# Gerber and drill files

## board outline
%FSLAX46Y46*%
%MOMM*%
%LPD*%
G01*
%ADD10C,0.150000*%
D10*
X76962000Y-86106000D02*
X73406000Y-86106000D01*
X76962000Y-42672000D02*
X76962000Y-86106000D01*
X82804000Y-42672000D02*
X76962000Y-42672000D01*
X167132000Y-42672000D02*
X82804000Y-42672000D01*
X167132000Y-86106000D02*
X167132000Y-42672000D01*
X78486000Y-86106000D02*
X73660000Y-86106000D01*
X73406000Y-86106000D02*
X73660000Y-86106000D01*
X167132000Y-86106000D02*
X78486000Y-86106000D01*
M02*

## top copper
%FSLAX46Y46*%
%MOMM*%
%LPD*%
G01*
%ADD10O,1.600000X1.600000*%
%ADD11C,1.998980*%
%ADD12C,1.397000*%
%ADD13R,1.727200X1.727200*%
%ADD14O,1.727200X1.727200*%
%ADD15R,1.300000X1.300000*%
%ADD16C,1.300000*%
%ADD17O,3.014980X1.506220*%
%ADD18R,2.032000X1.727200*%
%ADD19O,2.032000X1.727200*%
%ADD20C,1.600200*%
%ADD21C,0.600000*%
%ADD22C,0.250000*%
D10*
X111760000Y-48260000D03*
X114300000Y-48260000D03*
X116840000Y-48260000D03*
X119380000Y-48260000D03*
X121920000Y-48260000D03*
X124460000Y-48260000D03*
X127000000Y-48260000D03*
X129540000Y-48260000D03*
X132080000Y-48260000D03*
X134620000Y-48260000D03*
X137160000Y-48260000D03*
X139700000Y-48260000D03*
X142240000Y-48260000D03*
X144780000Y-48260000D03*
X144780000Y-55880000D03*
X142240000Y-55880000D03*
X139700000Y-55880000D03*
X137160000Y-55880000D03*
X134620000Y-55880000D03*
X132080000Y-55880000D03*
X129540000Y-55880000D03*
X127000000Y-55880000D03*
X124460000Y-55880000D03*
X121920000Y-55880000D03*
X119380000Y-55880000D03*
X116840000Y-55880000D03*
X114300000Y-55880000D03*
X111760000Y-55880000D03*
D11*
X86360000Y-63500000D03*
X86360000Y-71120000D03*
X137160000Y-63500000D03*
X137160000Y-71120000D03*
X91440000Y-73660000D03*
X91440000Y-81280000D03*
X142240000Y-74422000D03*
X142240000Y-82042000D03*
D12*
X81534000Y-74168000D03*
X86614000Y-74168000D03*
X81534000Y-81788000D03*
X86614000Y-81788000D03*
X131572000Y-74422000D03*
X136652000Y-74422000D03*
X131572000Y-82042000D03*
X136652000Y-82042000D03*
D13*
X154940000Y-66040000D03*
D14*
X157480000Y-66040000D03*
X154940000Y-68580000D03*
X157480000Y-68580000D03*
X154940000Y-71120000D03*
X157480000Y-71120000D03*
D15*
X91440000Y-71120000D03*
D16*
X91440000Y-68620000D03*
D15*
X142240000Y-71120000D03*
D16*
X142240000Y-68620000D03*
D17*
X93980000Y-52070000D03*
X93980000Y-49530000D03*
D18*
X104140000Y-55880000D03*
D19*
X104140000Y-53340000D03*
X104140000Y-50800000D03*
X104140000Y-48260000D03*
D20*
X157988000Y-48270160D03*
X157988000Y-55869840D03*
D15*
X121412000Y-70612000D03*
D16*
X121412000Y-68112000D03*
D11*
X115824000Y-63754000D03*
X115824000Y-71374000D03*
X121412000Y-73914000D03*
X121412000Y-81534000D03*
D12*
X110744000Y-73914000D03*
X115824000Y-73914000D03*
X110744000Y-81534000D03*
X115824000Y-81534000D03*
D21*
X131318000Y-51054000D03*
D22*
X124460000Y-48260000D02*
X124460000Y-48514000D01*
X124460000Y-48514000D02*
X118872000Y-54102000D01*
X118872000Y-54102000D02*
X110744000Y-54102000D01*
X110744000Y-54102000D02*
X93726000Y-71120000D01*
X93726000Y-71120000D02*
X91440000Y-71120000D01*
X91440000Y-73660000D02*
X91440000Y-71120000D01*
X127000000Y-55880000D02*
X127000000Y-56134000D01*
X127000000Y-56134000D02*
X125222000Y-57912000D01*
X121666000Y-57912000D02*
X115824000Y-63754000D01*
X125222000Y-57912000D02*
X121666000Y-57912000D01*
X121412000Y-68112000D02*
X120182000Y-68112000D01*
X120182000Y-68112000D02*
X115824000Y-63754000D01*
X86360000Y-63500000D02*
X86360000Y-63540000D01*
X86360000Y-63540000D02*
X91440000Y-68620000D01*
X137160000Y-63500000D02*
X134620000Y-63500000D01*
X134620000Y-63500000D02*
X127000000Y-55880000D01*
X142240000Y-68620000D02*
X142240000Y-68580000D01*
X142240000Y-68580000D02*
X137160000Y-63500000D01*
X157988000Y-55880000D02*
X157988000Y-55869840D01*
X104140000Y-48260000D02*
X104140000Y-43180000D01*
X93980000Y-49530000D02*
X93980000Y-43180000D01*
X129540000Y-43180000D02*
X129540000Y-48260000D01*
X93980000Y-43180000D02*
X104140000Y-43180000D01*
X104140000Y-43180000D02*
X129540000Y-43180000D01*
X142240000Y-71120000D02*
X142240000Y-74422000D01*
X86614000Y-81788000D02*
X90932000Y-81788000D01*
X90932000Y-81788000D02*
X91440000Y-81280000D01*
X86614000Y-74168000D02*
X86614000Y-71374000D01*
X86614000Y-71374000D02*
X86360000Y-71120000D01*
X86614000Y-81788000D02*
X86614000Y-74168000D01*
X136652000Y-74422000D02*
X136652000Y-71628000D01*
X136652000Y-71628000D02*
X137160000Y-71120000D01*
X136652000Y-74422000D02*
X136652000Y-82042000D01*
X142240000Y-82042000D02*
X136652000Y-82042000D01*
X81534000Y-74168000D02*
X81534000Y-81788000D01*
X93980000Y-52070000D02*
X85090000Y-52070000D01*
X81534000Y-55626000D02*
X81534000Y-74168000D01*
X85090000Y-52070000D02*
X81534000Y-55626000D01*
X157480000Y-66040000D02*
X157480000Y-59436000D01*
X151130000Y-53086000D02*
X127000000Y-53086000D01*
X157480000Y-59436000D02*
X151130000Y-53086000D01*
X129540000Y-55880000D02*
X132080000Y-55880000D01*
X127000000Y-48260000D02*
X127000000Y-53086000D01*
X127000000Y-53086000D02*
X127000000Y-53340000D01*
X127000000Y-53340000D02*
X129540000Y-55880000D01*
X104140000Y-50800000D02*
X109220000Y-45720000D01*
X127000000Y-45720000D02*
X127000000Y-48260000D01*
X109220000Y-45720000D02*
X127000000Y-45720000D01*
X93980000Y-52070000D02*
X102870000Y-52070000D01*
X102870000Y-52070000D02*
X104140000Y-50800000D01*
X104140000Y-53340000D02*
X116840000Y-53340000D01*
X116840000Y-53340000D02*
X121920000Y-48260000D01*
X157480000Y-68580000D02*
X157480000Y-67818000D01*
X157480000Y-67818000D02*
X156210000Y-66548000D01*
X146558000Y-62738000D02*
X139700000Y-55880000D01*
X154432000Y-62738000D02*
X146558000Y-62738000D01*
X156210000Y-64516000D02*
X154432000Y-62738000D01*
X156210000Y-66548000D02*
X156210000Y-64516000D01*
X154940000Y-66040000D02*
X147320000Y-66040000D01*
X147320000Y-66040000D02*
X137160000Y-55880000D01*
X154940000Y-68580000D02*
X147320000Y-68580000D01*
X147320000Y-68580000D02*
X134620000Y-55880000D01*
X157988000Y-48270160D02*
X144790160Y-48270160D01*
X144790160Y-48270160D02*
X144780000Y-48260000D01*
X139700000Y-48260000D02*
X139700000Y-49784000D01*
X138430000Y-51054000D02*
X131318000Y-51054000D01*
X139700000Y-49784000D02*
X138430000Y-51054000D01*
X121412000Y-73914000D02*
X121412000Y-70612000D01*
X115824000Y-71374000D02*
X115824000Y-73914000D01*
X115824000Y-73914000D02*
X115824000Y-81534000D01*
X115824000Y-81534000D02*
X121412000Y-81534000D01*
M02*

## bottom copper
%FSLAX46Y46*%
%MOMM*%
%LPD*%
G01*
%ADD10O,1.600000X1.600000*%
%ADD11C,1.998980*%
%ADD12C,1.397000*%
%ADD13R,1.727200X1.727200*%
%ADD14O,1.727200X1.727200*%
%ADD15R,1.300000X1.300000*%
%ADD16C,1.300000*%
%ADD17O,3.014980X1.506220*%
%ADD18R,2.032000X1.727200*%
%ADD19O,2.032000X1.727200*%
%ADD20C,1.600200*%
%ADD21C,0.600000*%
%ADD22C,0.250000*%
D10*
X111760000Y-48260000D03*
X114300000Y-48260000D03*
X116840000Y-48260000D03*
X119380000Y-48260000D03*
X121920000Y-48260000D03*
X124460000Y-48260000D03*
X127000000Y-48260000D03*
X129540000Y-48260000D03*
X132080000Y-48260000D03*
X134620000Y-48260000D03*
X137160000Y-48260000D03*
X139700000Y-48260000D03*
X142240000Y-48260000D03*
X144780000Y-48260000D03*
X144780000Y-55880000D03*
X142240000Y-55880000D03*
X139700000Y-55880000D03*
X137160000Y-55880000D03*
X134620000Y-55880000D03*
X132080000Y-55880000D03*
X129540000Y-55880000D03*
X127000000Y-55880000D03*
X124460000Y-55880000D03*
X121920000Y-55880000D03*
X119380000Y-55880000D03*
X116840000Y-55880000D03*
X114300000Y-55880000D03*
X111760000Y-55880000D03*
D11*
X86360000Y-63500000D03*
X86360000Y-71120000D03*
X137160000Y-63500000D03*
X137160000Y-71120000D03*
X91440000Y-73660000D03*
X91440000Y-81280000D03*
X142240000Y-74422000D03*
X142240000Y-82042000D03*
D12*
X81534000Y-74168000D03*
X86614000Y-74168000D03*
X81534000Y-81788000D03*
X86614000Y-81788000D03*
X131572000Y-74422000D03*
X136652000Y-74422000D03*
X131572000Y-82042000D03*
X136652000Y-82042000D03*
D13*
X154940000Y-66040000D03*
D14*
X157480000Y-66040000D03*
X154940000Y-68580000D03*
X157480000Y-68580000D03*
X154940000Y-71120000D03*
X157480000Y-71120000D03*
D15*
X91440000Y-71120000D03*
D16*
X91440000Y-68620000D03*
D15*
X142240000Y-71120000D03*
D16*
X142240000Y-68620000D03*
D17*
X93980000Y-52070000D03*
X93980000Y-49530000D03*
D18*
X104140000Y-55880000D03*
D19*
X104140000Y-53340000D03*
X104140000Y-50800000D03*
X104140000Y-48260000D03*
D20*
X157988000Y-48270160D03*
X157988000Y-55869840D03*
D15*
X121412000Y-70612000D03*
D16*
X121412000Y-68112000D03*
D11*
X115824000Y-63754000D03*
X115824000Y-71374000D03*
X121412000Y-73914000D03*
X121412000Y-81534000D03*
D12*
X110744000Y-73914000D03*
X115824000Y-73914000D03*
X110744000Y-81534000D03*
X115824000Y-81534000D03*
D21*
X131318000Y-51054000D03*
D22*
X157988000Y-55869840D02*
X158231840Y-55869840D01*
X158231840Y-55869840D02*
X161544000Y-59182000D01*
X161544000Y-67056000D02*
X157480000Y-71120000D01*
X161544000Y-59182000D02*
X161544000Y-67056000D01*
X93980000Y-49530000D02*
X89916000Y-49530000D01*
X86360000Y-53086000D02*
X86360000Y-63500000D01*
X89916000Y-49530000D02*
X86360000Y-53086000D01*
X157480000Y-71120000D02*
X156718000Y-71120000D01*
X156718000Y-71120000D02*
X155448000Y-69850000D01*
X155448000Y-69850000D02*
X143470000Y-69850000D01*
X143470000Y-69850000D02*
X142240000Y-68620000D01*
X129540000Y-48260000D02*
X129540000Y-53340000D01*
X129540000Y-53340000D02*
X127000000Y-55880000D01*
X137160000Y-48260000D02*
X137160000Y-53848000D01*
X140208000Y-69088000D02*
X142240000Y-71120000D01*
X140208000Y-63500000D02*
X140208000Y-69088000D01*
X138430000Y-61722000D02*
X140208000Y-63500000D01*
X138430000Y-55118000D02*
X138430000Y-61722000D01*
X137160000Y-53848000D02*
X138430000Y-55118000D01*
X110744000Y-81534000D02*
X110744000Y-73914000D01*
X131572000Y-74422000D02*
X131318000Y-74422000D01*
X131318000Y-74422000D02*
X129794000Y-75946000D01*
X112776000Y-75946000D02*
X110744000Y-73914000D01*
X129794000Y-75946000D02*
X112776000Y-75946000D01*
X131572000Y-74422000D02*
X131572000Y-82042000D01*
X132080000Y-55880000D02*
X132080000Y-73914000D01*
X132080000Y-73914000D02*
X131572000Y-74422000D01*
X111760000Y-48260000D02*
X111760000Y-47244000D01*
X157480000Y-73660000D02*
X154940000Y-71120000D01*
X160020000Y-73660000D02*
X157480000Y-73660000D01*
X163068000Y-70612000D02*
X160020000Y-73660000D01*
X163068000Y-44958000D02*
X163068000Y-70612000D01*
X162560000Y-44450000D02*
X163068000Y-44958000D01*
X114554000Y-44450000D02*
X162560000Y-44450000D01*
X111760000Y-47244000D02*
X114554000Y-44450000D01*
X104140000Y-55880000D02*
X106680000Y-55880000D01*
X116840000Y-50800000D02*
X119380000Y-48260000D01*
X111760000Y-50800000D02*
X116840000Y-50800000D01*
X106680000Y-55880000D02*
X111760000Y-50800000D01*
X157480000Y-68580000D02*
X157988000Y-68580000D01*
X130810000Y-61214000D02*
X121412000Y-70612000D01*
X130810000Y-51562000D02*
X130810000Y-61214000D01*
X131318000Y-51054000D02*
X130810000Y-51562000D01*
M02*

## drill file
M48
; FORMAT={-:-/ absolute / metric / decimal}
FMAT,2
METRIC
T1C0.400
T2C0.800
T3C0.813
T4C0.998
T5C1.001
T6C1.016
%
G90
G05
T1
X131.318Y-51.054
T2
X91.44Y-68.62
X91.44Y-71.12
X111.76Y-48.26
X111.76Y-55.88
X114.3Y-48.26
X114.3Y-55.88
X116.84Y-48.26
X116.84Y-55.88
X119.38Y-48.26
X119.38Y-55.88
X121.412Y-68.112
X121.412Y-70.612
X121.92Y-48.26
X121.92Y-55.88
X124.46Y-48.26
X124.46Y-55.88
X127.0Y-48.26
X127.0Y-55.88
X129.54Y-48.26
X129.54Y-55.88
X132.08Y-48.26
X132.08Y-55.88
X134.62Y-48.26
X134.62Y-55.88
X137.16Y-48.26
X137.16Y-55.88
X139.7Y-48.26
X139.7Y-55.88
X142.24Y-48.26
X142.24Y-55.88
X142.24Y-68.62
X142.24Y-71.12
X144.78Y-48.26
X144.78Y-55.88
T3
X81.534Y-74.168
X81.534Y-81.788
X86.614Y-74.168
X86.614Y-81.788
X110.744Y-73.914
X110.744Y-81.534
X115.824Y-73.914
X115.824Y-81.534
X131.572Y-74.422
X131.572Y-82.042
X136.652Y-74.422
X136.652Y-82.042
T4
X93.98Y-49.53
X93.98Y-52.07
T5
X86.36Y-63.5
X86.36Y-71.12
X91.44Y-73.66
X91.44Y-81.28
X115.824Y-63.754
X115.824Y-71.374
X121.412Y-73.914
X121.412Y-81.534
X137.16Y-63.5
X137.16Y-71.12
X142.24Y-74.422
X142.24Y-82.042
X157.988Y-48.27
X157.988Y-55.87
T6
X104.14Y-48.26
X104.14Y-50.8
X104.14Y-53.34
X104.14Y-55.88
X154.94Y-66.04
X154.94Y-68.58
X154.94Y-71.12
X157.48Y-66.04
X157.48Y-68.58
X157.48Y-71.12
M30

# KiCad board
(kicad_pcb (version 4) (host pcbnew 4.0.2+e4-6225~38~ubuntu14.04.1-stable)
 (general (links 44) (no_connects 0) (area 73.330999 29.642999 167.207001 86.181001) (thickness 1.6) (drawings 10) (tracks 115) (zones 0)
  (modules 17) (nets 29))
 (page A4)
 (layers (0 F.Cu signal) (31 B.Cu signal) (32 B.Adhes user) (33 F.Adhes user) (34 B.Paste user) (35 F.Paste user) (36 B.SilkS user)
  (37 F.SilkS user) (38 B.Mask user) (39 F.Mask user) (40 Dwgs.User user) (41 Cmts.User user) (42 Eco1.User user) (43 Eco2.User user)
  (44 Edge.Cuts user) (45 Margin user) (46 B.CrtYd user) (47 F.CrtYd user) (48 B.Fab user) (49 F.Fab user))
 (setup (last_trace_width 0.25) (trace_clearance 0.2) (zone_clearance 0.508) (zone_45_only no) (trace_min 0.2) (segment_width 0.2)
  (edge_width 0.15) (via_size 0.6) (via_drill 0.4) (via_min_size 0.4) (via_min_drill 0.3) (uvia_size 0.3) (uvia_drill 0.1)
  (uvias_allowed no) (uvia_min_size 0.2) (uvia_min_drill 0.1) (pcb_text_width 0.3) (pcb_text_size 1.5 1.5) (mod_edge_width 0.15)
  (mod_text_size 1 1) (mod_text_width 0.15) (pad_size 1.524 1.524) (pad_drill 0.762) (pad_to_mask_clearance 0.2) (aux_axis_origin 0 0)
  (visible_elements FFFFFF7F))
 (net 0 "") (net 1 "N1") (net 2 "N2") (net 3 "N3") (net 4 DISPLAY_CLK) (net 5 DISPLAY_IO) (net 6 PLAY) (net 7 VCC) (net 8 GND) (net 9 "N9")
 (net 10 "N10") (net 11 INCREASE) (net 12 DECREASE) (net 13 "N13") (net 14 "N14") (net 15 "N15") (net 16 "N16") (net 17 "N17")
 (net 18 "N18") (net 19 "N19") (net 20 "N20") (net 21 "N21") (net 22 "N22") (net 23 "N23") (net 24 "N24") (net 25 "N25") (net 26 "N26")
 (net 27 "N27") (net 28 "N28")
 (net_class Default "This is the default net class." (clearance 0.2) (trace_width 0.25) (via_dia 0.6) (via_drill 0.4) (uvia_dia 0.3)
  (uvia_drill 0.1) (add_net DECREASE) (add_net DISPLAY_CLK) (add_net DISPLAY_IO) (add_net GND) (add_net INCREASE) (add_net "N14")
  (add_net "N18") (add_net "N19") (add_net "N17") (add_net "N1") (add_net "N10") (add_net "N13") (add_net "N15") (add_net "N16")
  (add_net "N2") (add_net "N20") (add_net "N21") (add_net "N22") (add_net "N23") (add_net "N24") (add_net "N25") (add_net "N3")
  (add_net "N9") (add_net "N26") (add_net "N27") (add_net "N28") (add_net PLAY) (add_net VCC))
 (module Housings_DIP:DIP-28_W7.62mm (layer B.Cu) (at 111.76 48.26 270)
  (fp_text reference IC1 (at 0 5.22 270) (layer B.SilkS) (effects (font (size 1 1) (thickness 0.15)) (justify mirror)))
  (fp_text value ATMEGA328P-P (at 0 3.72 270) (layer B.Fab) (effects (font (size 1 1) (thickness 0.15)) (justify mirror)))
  (pad 1 thru_hole oval (at 0 0 270) (size 1.6 1.6) (drill 0.8) (layers *.Cu *.Mask B.SilkS) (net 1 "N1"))
  (pad 2 thru_hole oval (at 0 -2.54 270) (size 1.6 1.6) (drill 0.8) (layers *.Cu *.Mask B.SilkS) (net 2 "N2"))
  (pad 3 thru_hole oval (at 0 -5.08 270) (size 1.6 1.6) (drill 0.8) (layers *.Cu *.Mask B.SilkS) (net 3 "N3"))
  (pad 4 thru_hole oval (at 0 -7.62 270) (size 1.6 1.6) (drill 0.8) (layers *.Cu *.Mask B.SilkS) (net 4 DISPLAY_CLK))
  (pad 5 thru_hole oval (at 0 -10.16 270) (size 1.6 1.6) (drill 0.8) (layers *.Cu *.Mask B.SilkS) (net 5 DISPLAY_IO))
  (pad 6 thru_hole oval (at 0 -12.7 270) (size 1.6 1.6) (drill 0.8) (layers *.Cu *.Mask B.SilkS) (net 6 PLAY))
  (pad 7 thru_hole oval (at 0 -15.24 270) (size 1.6 1.6) (drill 0.8) (layers *.Cu *.Mask B.SilkS) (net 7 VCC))
  (pad 8 thru_hole oval (at 0 -17.78 270) (size 1.6 1.6) (drill 0.8) (layers *.Cu *.Mask B.SilkS) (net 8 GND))
  (pad 9 thru_hole oval (at 0 -20.32 270) (size 1.6 1.6) (drill 0.8) (layers *.Cu *.Mask B.SilkS) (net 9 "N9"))
  (pad 10 thru_hole oval (at 0 -22.86 270) (size 1.6 1.6) (drill 0.8) (layers *.Cu *.Mask B.SilkS) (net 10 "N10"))
  (pad 11 thru_hole oval (at 0 -25.4 270) (size 1.6 1.6) (drill 0.8) (layers *.Cu *.Mask B.SilkS) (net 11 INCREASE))
  (pad 12 thru_hole oval (at 0 -27.94 270) (size 1.6 1.6) (drill 0.8) (layers *.Cu *.Mask B.SilkS) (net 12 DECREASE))
  (pad 13 thru_hole oval (at 0 -30.48 270) (size 1.6 1.6) (drill 0.8) (layers *.Cu *.Mask B.SilkS) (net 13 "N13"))
  (pad 14 thru_hole oval (at 0 -33.02 270) (size 1.6 1.6) (drill 0.8) (layers *.Cu *.Mask B.SilkS) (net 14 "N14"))
  (pad 15 thru_hole oval (at 7.62 -33.02 270) (size 1.6 1.6) (drill 0.8) (layers *.Cu *.Mask B.SilkS) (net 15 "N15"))
  (pad 16 thru_hole oval (at 7.62 -30.48 270) (size 1.6 1.6) (drill 0.8) (layers *.Cu *.Mask B.SilkS) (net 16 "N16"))
  (pad 17 thru_hole oval (at 7.62 -27.94 270) (size 1.6 1.6) (drill 0.8) (layers *.Cu *.Mask B.SilkS) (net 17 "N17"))
  (pad 18 thru_hole oval (at 7.62 -25.4 270) (size 1.6 1.6) (drill 0.8) (layers *.Cu *.Mask B.SilkS) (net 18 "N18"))
  (pad 19 thru_hole oval (at 7.62 -22.86 270) (size 1.6 1.6) (drill 0.8) (layers *.Cu *.Mask B.SilkS) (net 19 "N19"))
  (pad 20 thru_hole oval (at 7.62 -20.32 270) (size 1.6 1.6) (drill 0.8) (layers *.Cu *.Mask B.SilkS) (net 7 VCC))
  (pad 21 thru_hole oval (at 7.62 -17.78 270) (size 1.6 1.6) (drill 0.8) (layers *.Cu *.Mask B.SilkS) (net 7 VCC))
  (pad 22 thru_hole oval (at 7.62 -15.24 270) (size 1.6 1.6) (drill 0.8) (layers *.Cu *.Mask B.SilkS) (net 8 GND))
  (pad 23 thru_hole oval (at 7.62 -12.7 270) (size 1.6 1.6) (drill 0.8) (layers *.Cu *.Mask B.SilkS) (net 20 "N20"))
  (pad 24 thru_hole oval (at 7.62 -10.16 270) (size 1.6 1.6) (drill 0.8) (layers *.Cu *.Mask B.SilkS) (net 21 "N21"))
  (pad 25 thru_hole oval (at 7.62 -7.62 270) (size 1.6 1.6) (drill 0.8) (layers *.Cu *.Mask B.SilkS) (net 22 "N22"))
  (pad 26 thru_hole oval (at 7.62 -5.08 270) (size 1.6 1.6) (drill 0.8) (layers *.Cu *.Mask B.SilkS) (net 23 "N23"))
  (pad 27 thru_hole oval (at 7.62 -2.54 270) (size 1.6 1.6) (drill 0.8) (layers *.Cu *.Mask B.SilkS) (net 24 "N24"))
  (pad 28 thru_hole oval (at 7.62 0 270) (size 1.6 1.6) (drill 0.8) (layers *.Cu *.Mask B.SilkS) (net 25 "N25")))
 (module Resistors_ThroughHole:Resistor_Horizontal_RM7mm (layer F.Cu) (at 86.36 63.5 270)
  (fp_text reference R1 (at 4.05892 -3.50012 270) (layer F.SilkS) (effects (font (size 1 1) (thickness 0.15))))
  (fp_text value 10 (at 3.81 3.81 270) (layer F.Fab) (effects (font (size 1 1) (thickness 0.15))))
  (pad 1 thru_hole circle (at 0 0 270) (size 1.99898 1.99898) (drill 1.00076) (layers *.Cu *.SilkS *.Mask) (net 8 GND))
  (pad 2 thru_hole circle (at 7.62 0 270) (size 1.99898 1.99898) (drill 1.00076) (layers *.Cu *.SilkS *.Mask) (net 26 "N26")))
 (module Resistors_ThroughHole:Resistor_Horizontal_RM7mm (layer F.Cu) (at 137.16 63.5 270)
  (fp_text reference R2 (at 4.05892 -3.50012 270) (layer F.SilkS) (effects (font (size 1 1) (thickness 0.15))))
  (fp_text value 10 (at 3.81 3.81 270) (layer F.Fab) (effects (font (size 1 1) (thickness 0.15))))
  (pad 1 thru_hole circle (at 0 0 270) (size 1.99898 1.99898) (drill 1.00076) (layers *.Cu *.SilkS *.Mask) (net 8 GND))
  (pad 2 thru_hole circle (at 7.62 0 270) (size 1.99898 1.99898) (drill 1.00076) (layers *.Cu *.SilkS *.Mask) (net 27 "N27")))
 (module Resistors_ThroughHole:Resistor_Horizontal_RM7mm (layer B.Cu) (at 91.44 73.66 270)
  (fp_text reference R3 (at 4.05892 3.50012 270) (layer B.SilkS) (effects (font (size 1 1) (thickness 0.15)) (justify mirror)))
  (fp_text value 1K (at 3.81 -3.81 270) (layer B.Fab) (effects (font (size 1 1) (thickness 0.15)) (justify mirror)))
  (pad 1 thru_hole circle (at 0 0 270) (size 1.99898 1.99898) (drill 1.00076) (layers *.Cu *.SilkS *.Mask) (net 6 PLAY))
  (pad 2 thru_hole circle (at 7.62 0 270) (size 1.99898 1.99898) (drill 1.00076) (layers *.Cu *.SilkS *.Mask) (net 26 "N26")))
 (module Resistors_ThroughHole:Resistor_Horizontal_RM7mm (layer F.Cu) (at 142.24 74.422 270)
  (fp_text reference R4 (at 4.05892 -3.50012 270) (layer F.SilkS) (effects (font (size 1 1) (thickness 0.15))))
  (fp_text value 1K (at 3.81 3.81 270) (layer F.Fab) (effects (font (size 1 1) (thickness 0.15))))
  (pad 1 thru_hole circle (at 0 0 270) (size 1.99898 1.99898) (drill 1.00076) (layers *.Cu *.SilkS *.Mask) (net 11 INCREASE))
  (pad 2 thru_hole circle (at 7.62 0 270) (size 1.99898 1.99898) (drill 1.00076) (layers *.Cu *.SilkS *.Mask) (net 27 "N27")))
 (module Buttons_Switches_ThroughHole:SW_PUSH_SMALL (layer F.Cu) (at 84.074 77.978 90)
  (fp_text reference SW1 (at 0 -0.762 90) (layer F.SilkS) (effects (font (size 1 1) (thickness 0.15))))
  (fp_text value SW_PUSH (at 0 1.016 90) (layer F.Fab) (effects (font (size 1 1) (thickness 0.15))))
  (pad 1 thru_hole circle (at 3.81 -2.54 90) (size 1.397 1.397) (drill 0.8128) (layers *.Cu *.Mask F.SilkS) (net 7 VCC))
  (pad 2 thru_hole circle (at 3.81 2.54 90) (size 1.397 1.397) (drill 0.8128) (layers *.Cu *.Mask F.SilkS) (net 26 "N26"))
  (pad 1 thru_hole circle (at -3.81 -2.54 90) (size 1.397 1.397) (drill 0.8128) (layers *.Cu *.Mask F.SilkS) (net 7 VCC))
  (pad 2 thru_hole circle (at -3.81 2.54 90) (size 1.397 1.397) (drill 0.8128) (layers *.Cu *.Mask F.SilkS) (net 26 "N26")))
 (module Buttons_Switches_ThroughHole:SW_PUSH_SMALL (layer F.Cu) (at 134.112 78.232 90)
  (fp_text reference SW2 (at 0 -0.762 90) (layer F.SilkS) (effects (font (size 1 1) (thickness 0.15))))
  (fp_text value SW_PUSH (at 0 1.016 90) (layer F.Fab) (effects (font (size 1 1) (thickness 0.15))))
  (pad 1 thru_hole circle (at 3.81 -2.54 90) (size 1.397 1.397) (drill 0.8128) (layers *.Cu *.Mask F.SilkS) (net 7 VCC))
  (pad 2 thru_hole circle (at 3.81 2.54 90) (size 1.397 1.397) (drill 0.8128) (layers *.Cu *.Mask F.SilkS) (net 27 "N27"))
  (pad 1 thru_hole circle (at -3.81 -2.54 90) (size 1.397 1.397) (drill 0.8128) (layers *.Cu *.Mask F.SilkS) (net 7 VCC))
  (pad 2 thru_hole circle (at -3.81 2.54 90) (size 1.397 1.397) (drill 0.8128) (layers *.Cu *.Mask F.SilkS) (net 27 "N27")))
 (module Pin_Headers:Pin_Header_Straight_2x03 (layer F.Cu) (at 154.94 66.04)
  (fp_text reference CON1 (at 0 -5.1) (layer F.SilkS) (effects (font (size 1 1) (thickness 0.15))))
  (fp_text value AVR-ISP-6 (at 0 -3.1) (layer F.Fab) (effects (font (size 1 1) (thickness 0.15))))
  (pad 1 thru_hole rect (at 0 0) (size 1.7272 1.7272) (drill 1.016) (layers *.Cu *.Mask F.SilkS) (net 18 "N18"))
  (pad 2 thru_hole oval (at 2.54 0) (size 1.7272 1.7272) (drill 1.016) (layers *.Cu *.Mask F.SilkS) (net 7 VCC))
  (pad 3 thru_hole oval (at 0 2.54) (size 1.7272 1.7272) (drill 1.016) (layers *.Cu *.Mask F.SilkS) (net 19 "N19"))
  (pad 4 thru_hole oval (at 2.54 2.54) (size 1.7272 1.7272) (drill 1.016) (layers *.Cu *.Mask F.SilkS) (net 17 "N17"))
  (pad 5 thru_hole oval (at 0 5.08) (size 1.7272 1.7272) (drill 1.016) (layers *.Cu *.Mask F.SilkS) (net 1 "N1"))
  (pad 6 thru_hole oval (at 2.54 5.08) (size 1.7272 1.7272) (drill 1.016) (layers *.Cu *.Mask F.SilkS) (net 8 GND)))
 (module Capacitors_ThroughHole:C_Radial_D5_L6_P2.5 (layer B.Cu) (at 91.44 71.12 90)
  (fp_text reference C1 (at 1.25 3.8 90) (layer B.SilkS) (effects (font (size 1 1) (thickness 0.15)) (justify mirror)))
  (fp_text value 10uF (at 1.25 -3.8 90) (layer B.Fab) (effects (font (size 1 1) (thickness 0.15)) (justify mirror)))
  (pad 1 thru_hole rect (at 0 0 90) (size 1.3 1.3) (drill 0.8) (layers *.Cu *.Mask B.SilkS) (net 6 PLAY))
  (pad 2 thru_hole circle (at 2.5 0 90) (size 1.3 1.3) (drill 0.8) (layers *.Cu *.Mask B.SilkS) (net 8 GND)))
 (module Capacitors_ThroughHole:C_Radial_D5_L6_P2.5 (layer F.Cu) (at 142.24 71.12 90)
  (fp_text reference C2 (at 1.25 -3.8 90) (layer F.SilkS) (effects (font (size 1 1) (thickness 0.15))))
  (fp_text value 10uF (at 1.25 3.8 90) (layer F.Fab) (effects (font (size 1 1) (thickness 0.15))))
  (pad 1 thru_hole rect (at 0 0 90) (size 1.3 1.3) (drill 0.8) (layers *.Cu *.Mask F.SilkS) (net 11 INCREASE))
  (pad 2 thru_hole circle (at 2.5 0 90) (size 1.3 1.3) (drill 0.8) (layers *.Cu *.Mask F.SilkS) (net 8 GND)))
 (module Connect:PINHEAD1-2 (layer F.Cu) (at 93.98 50.8 90)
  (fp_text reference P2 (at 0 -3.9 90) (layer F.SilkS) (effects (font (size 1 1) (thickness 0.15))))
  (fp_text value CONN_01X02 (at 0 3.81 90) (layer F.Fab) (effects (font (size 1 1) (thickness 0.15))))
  (pad 1 thru_hole oval (at -1.27 0 90) (size 1.50622 3.01498) (drill 0.99822) (layers *.Cu *.Mask) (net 7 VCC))
  (pad 2 thru_hole oval (at 1.27 0 90) (size 1.50622 3.01498) (drill 0.99822) (layers *.Cu *.Mask) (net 8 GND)))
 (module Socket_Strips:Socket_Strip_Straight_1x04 (layer F.Cu) (at 104.14 55.88 90)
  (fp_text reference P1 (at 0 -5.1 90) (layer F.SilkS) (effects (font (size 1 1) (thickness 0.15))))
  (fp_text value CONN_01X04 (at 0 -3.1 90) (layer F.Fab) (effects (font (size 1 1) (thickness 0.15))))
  (pad 1 thru_hole rect (at 0 0 90) (size 1.7272 2.032) (drill 1.016) (layers *.Cu *.Mask F.SilkS) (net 4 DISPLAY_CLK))
  (pad 2 thru_hole oval (at 2.54 0 90) (size 1.7272 2.032) (drill 1.016) (layers *.Cu *.Mask F.SilkS) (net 5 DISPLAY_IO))
  (pad 3 thru_hole oval (at 5.08 0 90) (size 1.7272 2.032) (drill 1.016) (layers *.Cu *.Mask F.SilkS) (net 7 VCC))
  (pad 4 thru_hole oval (at 7.62 0 90) (size 1.7272 2.032) (drill 1.016) (layers *.Cu *.Mask F.SilkS) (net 8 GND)))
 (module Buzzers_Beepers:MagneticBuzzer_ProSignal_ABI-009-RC (layer F.Cu) (at 157.988 48.26 270)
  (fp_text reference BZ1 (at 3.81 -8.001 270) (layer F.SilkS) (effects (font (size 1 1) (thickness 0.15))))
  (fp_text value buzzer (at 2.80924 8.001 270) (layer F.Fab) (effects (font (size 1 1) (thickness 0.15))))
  (pad 1 thru_hole circle (at 0.01016 0 270) (size 1.6002 1.6002) (drill 1.00076) (layers *.Cu *.Mask F.SilkS) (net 14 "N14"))
  (pad 2 thru_hole circle (at 7.60984 0 270) (size 1.6002 1.6002) (drill 1.00076) (layers *.Cu *.Mask F.SilkS) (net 8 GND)))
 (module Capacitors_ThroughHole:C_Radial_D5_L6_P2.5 (layer F.Cu) (at 121.412 70.612 90)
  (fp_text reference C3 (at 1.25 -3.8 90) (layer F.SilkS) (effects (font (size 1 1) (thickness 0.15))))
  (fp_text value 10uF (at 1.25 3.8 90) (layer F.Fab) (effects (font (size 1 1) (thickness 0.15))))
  (pad 1 thru_hole rect (at 0 0 90) (size 1.3 1.3) (drill 0.8) (layers *.Cu *.Mask F.SilkS) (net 12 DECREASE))
  (pad 2 thru_hole circle (at 2.5 0 90) (size 1.3 1.3) (drill 0.8) (layers *.Cu *.Mask F.SilkS) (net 8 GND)))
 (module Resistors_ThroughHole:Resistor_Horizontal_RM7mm (layer F.Cu) (at 115.824 63.754 270)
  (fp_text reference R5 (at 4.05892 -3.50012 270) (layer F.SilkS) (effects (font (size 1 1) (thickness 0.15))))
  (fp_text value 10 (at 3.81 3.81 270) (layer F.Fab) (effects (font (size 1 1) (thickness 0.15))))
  (pad 1 thru_hole circle (at 0 0 270) (size 1.99898 1.99898) (drill 1.00076) (layers *.Cu *.SilkS *.Mask) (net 8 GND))
  (pad 2 thru_hole circle (at 7.62 0 270) (size 1.99898 1.99898) (drill 1.00076) (layers *.Cu *.SilkS *.Mask) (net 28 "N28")))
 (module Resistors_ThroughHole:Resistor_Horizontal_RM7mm (layer F.Cu) (at 121.412 73.914 270)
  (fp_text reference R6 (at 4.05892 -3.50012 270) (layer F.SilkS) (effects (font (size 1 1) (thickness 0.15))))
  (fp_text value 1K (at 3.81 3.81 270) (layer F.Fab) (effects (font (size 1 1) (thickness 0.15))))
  (pad 1 thru_hole circle (at 0 0 270) (size 1.99898 1.99898) (drill 1.00076) (layers *.Cu *.SilkS *.Mask) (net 12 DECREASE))
  (pad 2 thru_hole circle (at 7.62 0 270) (size 1.99898 1.99898) (drill 1.00076) (layers *.Cu *.SilkS *.Mask) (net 28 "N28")))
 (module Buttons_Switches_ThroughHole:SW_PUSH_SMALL (layer F.Cu) (at 113.284 77.724 90)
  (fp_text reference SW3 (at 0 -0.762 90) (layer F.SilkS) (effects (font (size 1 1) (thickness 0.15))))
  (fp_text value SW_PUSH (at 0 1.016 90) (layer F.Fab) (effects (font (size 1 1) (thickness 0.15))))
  (pad 1 thru_hole circle (at 3.81 -2.54 90) (size 1.397 1.397) (drill 0.8128) (layers *.Cu *.Mask F.SilkS) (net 7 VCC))
  (pad 2 thru_hole circle (at 3.81 2.54 90) (size 1.397 1.397) (drill 0.8128) (layers *.Cu *.Mask F.SilkS) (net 28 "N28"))
  (pad 1 thru_hole circle (at -3.81 -2.54 90) (size 1.397 1.397) (drill 0.8128) (layers *.Cu *.Mask F.SilkS) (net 7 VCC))
  (pad 2 thru_hole circle (at -3.81 2.54 90) (size 1.397 1.397) (drill 0.8128) (layers *.Cu *.Mask F.SilkS) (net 28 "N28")))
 (gr_line (start 76.962 86.106) (end 73.406 86.106) (angle 90) (layer Edge.Cuts) (width 0.15))
 (gr_line (start 76.962 42.672) (end 76.962 86.106) (angle 90) (layer Edge.Cuts) (width 0.15))
 (gr_line (start 82.804 42.672) (end 76.962 42.672) (angle 90) (layer Edge.Cuts) (width 0.15))
 (gr_line (start 167.132 42.672) (end 82.804 42.672) (angle 90) (layer Edge.Cuts) (width 0.15))
 (gr_line (start 167.132 86.106) (end 167.132 42.672) (angle 90) (layer Edge.Cuts) (width 0.15))
 (gr_line (start 78.486 86.106) (end 73.66 86.106) (angle 90) (layer Edge.Cuts) (width 0.15))
 (gr_line (start 73.406 86.106) (end 73.66 86.106) (angle 90) (layer Edge.Cuts) (width 0.15))
 (gr_line (start 167.132 86.106) (end 78.486 86.106) (angle 90) (layer Edge.Cuts) (width 0.15))
 (segment (start 124.46 48.26) (end 124.46 48.514) (width 0.25) (layer F.Cu) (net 6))
 (segment (start 124.46 48.514) (end 118.872 54.102) (width 0.25) (layer F.Cu) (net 6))
 (segment (start 118.872 54.102) (end 110.744 54.102) (width 0.25) (layer F.Cu) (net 6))
 (segment (start 110.744 54.102) (end 93.726 71.12) (width 0.25) (layer F.Cu) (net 6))
 (segment (start 93.726 71.12) (end 91.44 71.12) (width 0.25) (layer F.Cu) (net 6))
 (segment (start 91.44 73.66) (end 91.44 71.12) (width 0.25) (layer F.Cu) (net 6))
 (segment (start 157.988 55.86984) (end 158.23184 55.86984) (width 0.25) (layer B.Cu) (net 8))
 (segment (start 158.23184 55.86984) (end 161.544 59.182) (width 0.25) (layer B.Cu) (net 8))
 (segment (start 161.544 67.056) (end 157.48 71.12) (width 0.25) (layer B.Cu) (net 8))
 (segment (start 161.544 59.182) (end 161.544 67.056) (width 0.25) (layer B.Cu) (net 8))
 (segment (start 127 55.88) (end 127 56.134) (width 0.25) (layer F.Cu) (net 8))
 (segment (start 127 56.134) (end 125.222 57.912) (width 0.25) (layer F.Cu) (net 8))
 (segment (start 121.666 57.912) (end 115.824 63.754) (width 0.25) (layer F.Cu) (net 8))
 (segment (start 125.222 57.912) (end 121.666 57.912) (width 0.25) (layer F.Cu) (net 8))
 (segment (start 121.412 68.112) (end 120.182 68.112) (width 0.25) (layer F.Cu) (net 8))
 (segment (start 120.182 68.112) (end 115.824 63.754) (width 0.25) (layer F.Cu) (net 8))
 (segment (start 86.36 63.5) (end 86.36 63.54) (width 0.25) (layer F.Cu) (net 8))
 (segment (start 86.36 63.54) (end 91.44 68.62) (width 0.25) (layer F.Cu) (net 8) (status 20))
 (segment (start 93.98 49.53) (end 89.916 49.53) (width 0.25) (layer B.Cu) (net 8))
 (segment (start 86.36 53.086) (end 86.36 63.5) (width 0.25) (layer B.Cu) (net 8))
 (segment (start 89.916 49.53) (end 86.36 53.086) (width 0.25) (layer B.Cu) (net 8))
 (segment (start 157.48 71.12) (end 156.718 71.12) (width 0.25) (layer B.Cu) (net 8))
 (segment (start 156.718 71.12) (end 155.448 69.85) (width 0.25) (layer B.Cu) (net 8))
 (segment (start 155.448 69.85) (end 143.47 69.85) (width 0.25) (layer B.Cu) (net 8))
 (segment (start 143.47 69.85) (end 142.24 68.62) (width 0.25) (layer B.Cu) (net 8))
 (segment (start 137.16 63.5) (end 134.62 63.5) (width 0.25) (layer F.Cu) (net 8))
 (segment (start 134.62 63.5) (end 127 55.88) (width 0.25) (layer F.Cu) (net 8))
 (segment (start 142.24 68.62) (end 142.24 68.58) (width 0.25) (layer F.Cu) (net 8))
 (segment (start 142.24 68.58) (end 137.16 63.5) (width 0.25) (layer F.Cu) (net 8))
 (segment (start 129.54 48.26) (end 129.54 53.34) (width 0.25) (layer B.Cu) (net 8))
 (segment (start 129.54 53.34) (end 127 55.88) (width 0.25) (layer B.Cu) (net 8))
 (segment (start 157.988 55.88) (end 157.988 55.86984) (width 0.25) (layer F.Cu) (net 8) (status 30))
 (segment (start 104.14 48.26) (end 104.14 43.18) (width 0.25) (layer F.Cu) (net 8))
 (segment (start 93.98 49.53) (end 93.98 43.18) (width 0.25) (layer F.Cu) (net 8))
 (segment (start 129.54 43.18) (end 129.54 48.26) (width 0.25) (layer F.Cu) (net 8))
 (segment (start 93.98 43.18) (end 104.14 43.18) (width 0.25) (layer F.Cu) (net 8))
 (segment (start 104.14 43.18) (end 129.54 43.18) (width 0.25) (layer F.Cu) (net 8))
 (segment (start 142.24 71.12) (end 142.24 74.422) (width 0.25) (layer F.Cu) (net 11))
 (segment (start 137.16 48.26) (end 137.16 53.848) (width 0.25) (layer B.Cu) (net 11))
 (segment (start 140.208 69.088) (end 142.24 71.12) (width 0.25) (layer B.Cu) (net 11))
 (segment (start 140.208 63.5) (end 140.208 69.088) (width 0.25) (layer B.Cu) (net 11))
 (segment (start 138.43 61.722) (end 140.208 63.5) (width 0.25) (layer B.Cu) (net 11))
 (segment (start 138.43 55.118) (end 138.43 61.722) (width 0.25) (layer B.Cu) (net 11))
 (segment (start 137.16 53.848) (end 138.43 55.118) (width 0.25) (layer B.Cu) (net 11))
 (segment (start 86.614 81.788) (end 90.932 81.788) (width 0.25) (layer F.Cu) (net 26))
 (segment (start 90.932 81.788) (end 91.44 81.28) (width 0.25) (layer F.Cu) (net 26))
 (segment (start 86.614 74.168) (end 86.614 71.374) (width 0.25) (layer F.Cu) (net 26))
 (segment (start 86.614 71.374) (end 86.36 71.12) (width 0.25) (layer F.Cu) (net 26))
 (segment (start 86.614 81.788) (end 86.614 74.168) (width 0.25) (layer F.Cu) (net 26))
 (segment (start 136.652 74.422) (end 136.652 71.628) (width 0.25) (layer F.Cu) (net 27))
 (segment (start 136.652 71.628) (end 137.16 71.12) (width 0.25) (layer F.Cu) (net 27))
 (segment (start 136.652 74.422) (end 136.652 82.042) (width 0.25) (layer F.Cu) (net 27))
 (segment (start 142.24 82.042) (end 136.652 82.042) (width 0.25) (layer F.Cu) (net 27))
 (segment (start 110.744 81.534) (end 110.744 73.914) (width 0.25) (layer B.Cu) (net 7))
 (segment (start 131.572 74.422) (end 131.318 74.422) (width 0.25) (layer B.Cu) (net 7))
 (segment (start 131.318 74.422) (end 129.794 75.946) (width 0.25) (layer B.Cu) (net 7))
 (segment (start 112.776 75.946) (end 110.744 73.914) (width 0.25) (layer B.Cu) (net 7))
 (segment (start 129.794 75.946) (end 112.776 75.946) (width 0.25) (layer B.Cu) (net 7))
 (segment (start 81.534 74.168) (end 81.534 81.788) (width 0.25) (layer F.Cu) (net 7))
 (segment (start 93.98 52.07) (end 85.09 52.07) (width 0.25) (layer F.Cu) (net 7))
 (segment (start 81.534 55.626) (end 81.534 74.168) (width 0.25) (layer F.Cu) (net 7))
 (segment (start 85.09 52.07) (end 81.534 55.626) (width 0.25) (layer F.Cu) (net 7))
 (segment (start 131.572 74.422) (end 131.572 82.042) (width 0.25) (layer B.Cu) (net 7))
 (segment (start 157.48 66.04) (end 157.48 59.436) (width 0.25) (layer F.Cu) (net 7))
 (segment (start 151.13 53.086) (end 127 53.086) (width 0.25) (layer F.Cu) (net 7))
 (segment (start 157.48 59.436) (end 151.13 53.086) (width 0.25) (layer F.Cu) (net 7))
 (segment (start 132.08 55.88) (end 132.08 73.914) (width 0.25) (layer B.Cu) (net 7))
 (segment (start 132.08 73.914) (end 131.572 74.422) (width 0.25) (layer B.Cu) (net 7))
 (segment (start 129.54 55.88) (end 132.08 55.88) (width 0.25) (layer F.Cu) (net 7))
 (segment (start 127 48.26) (end 127 53.086) (width 0.25) (layer F.Cu) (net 7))
 (segment (start 127 53.086) (end 127 53.34) (width 0.25) (layer F.Cu) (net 7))
 (segment (start 127 53.34) (end 129.54 55.88) (width 0.25) (layer F.Cu) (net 7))
 (segment (start 104.14 50.8) (end 109.22 45.72) (width 0.25) (layer F.Cu) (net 7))
 (segment (start 127 45.72) (end 127 48.26) (width 0.25) (layer F.Cu) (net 7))
 (segment (start 109.22 45.72) (end 127 45.72) (width 0.25) (layer F.Cu) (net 7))
 (segment (start 93.98 52.07) (end 102.87 52.07) (width 0.25) (layer F.Cu) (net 7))
 (segment (start 102.87 52.07) (end 104.14 50.8) (width 0.25) (layer F.Cu) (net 7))
 (segment (start 111.76 48.26) (end 111.76 47.244) (width 0.25) (layer B.Cu) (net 1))
 (segment (start 157.48 73.66) (end 154.94 71.12) (width 0.25) (layer B.Cu) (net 1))
 (segment (start 160.02 73.66) (end 157.48 73.66) (width 0.25) (layer B.Cu) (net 1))
 (segment (start 163.068 70.612) (end 160.02 73.66) (width 0.25) (layer B.Cu) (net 1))
 (segment (start 163.068 44.958) (end 163.068 70.612) (width 0.25) (layer B.Cu) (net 1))
 (segment (start 162.56 44.45) (end 163.068 44.958) (width 0.25) (layer B.Cu) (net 1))
 (segment (start 114.554 44.45) (end 162.56 44.45) (width 0.25) (layer B.Cu) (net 1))
 (segment (start 111.76 47.244) (end 114.554 44.45) (width 0.25) (layer B.Cu) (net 1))
 (segment (start 104.14 55.88) (end 106.68 55.88) (width 0.25) (layer B.Cu) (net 4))
 (segment (start 116.84 50.8) (end 119.38 48.26) (width 0.25) (layer B.Cu) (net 4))
 (segment (start 111.76 50.8) (end 116.84 50.8) (width 0.25) (layer B.Cu) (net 4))
 (segment (start 106.68 55.88) (end 111.76 50.8) (width 0.25) (layer B.Cu) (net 4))
 (segment (start 104.14 53.34) (end 116.84 53.34) (width 0.25) (layer F.Cu) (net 5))
 (segment (start 116.84 53.34) (end 121.92 48.26) (width 0.25) (layer F.Cu) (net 5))
 (segment (start 157.48 68.58) (end 157.48 67.818) (width 0.25) (layer F.Cu) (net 17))
 (segment (start 157.48 67.818) (end 156.21 66.548) (width 0.25) (layer F.Cu) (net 17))
 (segment (start 146.558 62.738) (end 139.7 55.88) (width 0.25) (layer F.Cu) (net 17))
 (segment (start 154.432 62.738) (end 146.558 62.738) (width 0.25) (layer F.Cu) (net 17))
 (segment (start 156.21 64.516) (end 154.432 62.738) (width 0.25) (layer F.Cu) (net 17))
 (segment (start 156.21 66.548) (end 156.21 64.516) (width 0.25) (layer F.Cu) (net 17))
 (segment (start 157.48 68.58) (end 157.988 68.58) (width 0.25) (layer B.Cu) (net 17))
 (segment (start 154.94 66.04) (end 147.32 66.04) (width 0.25) (layer F.Cu) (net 18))
 (segment (start 147.32 66.04) (end 137.16 55.88) (width 0.25) (layer F.Cu) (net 18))
 (segment (start 154.94 68.58) (end 147.32 68.58) (width 0.25) (layer F.Cu) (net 19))
 (segment (start 147.32 68.58) (end 134.62 55.88) (width 0.25) (layer F.Cu) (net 19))
 (segment (start 157.988 48.27016) (end 144.79016 48.27016) (width 0.25) (layer F.Cu) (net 14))
 (segment (start 144.79016 48.27016) (end 144.78 48.26) (width 0.25) (layer F.Cu) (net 14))
 (segment (start 139.7 48.26) (end 139.7 49.784) (width 0.25) (layer F.Cu) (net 12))
 (segment (start 130.81 61.214) (end 121.412 70.612) (width 0.25) (layer B.Cu) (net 12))
 (segment (start 130.81 51.562) (end 130.81 61.214) (width 0.25) (layer B.Cu) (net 12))
 (segment (start 131.318 51.054) (end 130.81 51.562) (width 0.25) (layer B.Cu) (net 12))
 (via (at 131.318 51.054) (size 0.6) (drill 0.4) (layers F.Cu B.Cu) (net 12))
 (segment (start 138.43 51.054) (end 131.318 51.054) (width 0.25) (layer F.Cu) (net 12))
 (segment (start 139.7 49.784) (end 138.43 51.054) (width 0.25) (layer F.Cu) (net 12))
 (segment (start 121.412 73.914) (end 121.412 70.612) (width 0.25) (layer F.Cu) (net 12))
 (segment (start 115.824 71.374) (end 115.824 73.914) (width 0.25) (layer F.Cu) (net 28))
 (segment (start 115.824 73.914) (end 115.824 81.534) (width 0.25) (layer F.Cu) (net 28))
 (segment (start 115.824 81.534) (end 121.412 81.534) (width 0.25) (layer F.Cu) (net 28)))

